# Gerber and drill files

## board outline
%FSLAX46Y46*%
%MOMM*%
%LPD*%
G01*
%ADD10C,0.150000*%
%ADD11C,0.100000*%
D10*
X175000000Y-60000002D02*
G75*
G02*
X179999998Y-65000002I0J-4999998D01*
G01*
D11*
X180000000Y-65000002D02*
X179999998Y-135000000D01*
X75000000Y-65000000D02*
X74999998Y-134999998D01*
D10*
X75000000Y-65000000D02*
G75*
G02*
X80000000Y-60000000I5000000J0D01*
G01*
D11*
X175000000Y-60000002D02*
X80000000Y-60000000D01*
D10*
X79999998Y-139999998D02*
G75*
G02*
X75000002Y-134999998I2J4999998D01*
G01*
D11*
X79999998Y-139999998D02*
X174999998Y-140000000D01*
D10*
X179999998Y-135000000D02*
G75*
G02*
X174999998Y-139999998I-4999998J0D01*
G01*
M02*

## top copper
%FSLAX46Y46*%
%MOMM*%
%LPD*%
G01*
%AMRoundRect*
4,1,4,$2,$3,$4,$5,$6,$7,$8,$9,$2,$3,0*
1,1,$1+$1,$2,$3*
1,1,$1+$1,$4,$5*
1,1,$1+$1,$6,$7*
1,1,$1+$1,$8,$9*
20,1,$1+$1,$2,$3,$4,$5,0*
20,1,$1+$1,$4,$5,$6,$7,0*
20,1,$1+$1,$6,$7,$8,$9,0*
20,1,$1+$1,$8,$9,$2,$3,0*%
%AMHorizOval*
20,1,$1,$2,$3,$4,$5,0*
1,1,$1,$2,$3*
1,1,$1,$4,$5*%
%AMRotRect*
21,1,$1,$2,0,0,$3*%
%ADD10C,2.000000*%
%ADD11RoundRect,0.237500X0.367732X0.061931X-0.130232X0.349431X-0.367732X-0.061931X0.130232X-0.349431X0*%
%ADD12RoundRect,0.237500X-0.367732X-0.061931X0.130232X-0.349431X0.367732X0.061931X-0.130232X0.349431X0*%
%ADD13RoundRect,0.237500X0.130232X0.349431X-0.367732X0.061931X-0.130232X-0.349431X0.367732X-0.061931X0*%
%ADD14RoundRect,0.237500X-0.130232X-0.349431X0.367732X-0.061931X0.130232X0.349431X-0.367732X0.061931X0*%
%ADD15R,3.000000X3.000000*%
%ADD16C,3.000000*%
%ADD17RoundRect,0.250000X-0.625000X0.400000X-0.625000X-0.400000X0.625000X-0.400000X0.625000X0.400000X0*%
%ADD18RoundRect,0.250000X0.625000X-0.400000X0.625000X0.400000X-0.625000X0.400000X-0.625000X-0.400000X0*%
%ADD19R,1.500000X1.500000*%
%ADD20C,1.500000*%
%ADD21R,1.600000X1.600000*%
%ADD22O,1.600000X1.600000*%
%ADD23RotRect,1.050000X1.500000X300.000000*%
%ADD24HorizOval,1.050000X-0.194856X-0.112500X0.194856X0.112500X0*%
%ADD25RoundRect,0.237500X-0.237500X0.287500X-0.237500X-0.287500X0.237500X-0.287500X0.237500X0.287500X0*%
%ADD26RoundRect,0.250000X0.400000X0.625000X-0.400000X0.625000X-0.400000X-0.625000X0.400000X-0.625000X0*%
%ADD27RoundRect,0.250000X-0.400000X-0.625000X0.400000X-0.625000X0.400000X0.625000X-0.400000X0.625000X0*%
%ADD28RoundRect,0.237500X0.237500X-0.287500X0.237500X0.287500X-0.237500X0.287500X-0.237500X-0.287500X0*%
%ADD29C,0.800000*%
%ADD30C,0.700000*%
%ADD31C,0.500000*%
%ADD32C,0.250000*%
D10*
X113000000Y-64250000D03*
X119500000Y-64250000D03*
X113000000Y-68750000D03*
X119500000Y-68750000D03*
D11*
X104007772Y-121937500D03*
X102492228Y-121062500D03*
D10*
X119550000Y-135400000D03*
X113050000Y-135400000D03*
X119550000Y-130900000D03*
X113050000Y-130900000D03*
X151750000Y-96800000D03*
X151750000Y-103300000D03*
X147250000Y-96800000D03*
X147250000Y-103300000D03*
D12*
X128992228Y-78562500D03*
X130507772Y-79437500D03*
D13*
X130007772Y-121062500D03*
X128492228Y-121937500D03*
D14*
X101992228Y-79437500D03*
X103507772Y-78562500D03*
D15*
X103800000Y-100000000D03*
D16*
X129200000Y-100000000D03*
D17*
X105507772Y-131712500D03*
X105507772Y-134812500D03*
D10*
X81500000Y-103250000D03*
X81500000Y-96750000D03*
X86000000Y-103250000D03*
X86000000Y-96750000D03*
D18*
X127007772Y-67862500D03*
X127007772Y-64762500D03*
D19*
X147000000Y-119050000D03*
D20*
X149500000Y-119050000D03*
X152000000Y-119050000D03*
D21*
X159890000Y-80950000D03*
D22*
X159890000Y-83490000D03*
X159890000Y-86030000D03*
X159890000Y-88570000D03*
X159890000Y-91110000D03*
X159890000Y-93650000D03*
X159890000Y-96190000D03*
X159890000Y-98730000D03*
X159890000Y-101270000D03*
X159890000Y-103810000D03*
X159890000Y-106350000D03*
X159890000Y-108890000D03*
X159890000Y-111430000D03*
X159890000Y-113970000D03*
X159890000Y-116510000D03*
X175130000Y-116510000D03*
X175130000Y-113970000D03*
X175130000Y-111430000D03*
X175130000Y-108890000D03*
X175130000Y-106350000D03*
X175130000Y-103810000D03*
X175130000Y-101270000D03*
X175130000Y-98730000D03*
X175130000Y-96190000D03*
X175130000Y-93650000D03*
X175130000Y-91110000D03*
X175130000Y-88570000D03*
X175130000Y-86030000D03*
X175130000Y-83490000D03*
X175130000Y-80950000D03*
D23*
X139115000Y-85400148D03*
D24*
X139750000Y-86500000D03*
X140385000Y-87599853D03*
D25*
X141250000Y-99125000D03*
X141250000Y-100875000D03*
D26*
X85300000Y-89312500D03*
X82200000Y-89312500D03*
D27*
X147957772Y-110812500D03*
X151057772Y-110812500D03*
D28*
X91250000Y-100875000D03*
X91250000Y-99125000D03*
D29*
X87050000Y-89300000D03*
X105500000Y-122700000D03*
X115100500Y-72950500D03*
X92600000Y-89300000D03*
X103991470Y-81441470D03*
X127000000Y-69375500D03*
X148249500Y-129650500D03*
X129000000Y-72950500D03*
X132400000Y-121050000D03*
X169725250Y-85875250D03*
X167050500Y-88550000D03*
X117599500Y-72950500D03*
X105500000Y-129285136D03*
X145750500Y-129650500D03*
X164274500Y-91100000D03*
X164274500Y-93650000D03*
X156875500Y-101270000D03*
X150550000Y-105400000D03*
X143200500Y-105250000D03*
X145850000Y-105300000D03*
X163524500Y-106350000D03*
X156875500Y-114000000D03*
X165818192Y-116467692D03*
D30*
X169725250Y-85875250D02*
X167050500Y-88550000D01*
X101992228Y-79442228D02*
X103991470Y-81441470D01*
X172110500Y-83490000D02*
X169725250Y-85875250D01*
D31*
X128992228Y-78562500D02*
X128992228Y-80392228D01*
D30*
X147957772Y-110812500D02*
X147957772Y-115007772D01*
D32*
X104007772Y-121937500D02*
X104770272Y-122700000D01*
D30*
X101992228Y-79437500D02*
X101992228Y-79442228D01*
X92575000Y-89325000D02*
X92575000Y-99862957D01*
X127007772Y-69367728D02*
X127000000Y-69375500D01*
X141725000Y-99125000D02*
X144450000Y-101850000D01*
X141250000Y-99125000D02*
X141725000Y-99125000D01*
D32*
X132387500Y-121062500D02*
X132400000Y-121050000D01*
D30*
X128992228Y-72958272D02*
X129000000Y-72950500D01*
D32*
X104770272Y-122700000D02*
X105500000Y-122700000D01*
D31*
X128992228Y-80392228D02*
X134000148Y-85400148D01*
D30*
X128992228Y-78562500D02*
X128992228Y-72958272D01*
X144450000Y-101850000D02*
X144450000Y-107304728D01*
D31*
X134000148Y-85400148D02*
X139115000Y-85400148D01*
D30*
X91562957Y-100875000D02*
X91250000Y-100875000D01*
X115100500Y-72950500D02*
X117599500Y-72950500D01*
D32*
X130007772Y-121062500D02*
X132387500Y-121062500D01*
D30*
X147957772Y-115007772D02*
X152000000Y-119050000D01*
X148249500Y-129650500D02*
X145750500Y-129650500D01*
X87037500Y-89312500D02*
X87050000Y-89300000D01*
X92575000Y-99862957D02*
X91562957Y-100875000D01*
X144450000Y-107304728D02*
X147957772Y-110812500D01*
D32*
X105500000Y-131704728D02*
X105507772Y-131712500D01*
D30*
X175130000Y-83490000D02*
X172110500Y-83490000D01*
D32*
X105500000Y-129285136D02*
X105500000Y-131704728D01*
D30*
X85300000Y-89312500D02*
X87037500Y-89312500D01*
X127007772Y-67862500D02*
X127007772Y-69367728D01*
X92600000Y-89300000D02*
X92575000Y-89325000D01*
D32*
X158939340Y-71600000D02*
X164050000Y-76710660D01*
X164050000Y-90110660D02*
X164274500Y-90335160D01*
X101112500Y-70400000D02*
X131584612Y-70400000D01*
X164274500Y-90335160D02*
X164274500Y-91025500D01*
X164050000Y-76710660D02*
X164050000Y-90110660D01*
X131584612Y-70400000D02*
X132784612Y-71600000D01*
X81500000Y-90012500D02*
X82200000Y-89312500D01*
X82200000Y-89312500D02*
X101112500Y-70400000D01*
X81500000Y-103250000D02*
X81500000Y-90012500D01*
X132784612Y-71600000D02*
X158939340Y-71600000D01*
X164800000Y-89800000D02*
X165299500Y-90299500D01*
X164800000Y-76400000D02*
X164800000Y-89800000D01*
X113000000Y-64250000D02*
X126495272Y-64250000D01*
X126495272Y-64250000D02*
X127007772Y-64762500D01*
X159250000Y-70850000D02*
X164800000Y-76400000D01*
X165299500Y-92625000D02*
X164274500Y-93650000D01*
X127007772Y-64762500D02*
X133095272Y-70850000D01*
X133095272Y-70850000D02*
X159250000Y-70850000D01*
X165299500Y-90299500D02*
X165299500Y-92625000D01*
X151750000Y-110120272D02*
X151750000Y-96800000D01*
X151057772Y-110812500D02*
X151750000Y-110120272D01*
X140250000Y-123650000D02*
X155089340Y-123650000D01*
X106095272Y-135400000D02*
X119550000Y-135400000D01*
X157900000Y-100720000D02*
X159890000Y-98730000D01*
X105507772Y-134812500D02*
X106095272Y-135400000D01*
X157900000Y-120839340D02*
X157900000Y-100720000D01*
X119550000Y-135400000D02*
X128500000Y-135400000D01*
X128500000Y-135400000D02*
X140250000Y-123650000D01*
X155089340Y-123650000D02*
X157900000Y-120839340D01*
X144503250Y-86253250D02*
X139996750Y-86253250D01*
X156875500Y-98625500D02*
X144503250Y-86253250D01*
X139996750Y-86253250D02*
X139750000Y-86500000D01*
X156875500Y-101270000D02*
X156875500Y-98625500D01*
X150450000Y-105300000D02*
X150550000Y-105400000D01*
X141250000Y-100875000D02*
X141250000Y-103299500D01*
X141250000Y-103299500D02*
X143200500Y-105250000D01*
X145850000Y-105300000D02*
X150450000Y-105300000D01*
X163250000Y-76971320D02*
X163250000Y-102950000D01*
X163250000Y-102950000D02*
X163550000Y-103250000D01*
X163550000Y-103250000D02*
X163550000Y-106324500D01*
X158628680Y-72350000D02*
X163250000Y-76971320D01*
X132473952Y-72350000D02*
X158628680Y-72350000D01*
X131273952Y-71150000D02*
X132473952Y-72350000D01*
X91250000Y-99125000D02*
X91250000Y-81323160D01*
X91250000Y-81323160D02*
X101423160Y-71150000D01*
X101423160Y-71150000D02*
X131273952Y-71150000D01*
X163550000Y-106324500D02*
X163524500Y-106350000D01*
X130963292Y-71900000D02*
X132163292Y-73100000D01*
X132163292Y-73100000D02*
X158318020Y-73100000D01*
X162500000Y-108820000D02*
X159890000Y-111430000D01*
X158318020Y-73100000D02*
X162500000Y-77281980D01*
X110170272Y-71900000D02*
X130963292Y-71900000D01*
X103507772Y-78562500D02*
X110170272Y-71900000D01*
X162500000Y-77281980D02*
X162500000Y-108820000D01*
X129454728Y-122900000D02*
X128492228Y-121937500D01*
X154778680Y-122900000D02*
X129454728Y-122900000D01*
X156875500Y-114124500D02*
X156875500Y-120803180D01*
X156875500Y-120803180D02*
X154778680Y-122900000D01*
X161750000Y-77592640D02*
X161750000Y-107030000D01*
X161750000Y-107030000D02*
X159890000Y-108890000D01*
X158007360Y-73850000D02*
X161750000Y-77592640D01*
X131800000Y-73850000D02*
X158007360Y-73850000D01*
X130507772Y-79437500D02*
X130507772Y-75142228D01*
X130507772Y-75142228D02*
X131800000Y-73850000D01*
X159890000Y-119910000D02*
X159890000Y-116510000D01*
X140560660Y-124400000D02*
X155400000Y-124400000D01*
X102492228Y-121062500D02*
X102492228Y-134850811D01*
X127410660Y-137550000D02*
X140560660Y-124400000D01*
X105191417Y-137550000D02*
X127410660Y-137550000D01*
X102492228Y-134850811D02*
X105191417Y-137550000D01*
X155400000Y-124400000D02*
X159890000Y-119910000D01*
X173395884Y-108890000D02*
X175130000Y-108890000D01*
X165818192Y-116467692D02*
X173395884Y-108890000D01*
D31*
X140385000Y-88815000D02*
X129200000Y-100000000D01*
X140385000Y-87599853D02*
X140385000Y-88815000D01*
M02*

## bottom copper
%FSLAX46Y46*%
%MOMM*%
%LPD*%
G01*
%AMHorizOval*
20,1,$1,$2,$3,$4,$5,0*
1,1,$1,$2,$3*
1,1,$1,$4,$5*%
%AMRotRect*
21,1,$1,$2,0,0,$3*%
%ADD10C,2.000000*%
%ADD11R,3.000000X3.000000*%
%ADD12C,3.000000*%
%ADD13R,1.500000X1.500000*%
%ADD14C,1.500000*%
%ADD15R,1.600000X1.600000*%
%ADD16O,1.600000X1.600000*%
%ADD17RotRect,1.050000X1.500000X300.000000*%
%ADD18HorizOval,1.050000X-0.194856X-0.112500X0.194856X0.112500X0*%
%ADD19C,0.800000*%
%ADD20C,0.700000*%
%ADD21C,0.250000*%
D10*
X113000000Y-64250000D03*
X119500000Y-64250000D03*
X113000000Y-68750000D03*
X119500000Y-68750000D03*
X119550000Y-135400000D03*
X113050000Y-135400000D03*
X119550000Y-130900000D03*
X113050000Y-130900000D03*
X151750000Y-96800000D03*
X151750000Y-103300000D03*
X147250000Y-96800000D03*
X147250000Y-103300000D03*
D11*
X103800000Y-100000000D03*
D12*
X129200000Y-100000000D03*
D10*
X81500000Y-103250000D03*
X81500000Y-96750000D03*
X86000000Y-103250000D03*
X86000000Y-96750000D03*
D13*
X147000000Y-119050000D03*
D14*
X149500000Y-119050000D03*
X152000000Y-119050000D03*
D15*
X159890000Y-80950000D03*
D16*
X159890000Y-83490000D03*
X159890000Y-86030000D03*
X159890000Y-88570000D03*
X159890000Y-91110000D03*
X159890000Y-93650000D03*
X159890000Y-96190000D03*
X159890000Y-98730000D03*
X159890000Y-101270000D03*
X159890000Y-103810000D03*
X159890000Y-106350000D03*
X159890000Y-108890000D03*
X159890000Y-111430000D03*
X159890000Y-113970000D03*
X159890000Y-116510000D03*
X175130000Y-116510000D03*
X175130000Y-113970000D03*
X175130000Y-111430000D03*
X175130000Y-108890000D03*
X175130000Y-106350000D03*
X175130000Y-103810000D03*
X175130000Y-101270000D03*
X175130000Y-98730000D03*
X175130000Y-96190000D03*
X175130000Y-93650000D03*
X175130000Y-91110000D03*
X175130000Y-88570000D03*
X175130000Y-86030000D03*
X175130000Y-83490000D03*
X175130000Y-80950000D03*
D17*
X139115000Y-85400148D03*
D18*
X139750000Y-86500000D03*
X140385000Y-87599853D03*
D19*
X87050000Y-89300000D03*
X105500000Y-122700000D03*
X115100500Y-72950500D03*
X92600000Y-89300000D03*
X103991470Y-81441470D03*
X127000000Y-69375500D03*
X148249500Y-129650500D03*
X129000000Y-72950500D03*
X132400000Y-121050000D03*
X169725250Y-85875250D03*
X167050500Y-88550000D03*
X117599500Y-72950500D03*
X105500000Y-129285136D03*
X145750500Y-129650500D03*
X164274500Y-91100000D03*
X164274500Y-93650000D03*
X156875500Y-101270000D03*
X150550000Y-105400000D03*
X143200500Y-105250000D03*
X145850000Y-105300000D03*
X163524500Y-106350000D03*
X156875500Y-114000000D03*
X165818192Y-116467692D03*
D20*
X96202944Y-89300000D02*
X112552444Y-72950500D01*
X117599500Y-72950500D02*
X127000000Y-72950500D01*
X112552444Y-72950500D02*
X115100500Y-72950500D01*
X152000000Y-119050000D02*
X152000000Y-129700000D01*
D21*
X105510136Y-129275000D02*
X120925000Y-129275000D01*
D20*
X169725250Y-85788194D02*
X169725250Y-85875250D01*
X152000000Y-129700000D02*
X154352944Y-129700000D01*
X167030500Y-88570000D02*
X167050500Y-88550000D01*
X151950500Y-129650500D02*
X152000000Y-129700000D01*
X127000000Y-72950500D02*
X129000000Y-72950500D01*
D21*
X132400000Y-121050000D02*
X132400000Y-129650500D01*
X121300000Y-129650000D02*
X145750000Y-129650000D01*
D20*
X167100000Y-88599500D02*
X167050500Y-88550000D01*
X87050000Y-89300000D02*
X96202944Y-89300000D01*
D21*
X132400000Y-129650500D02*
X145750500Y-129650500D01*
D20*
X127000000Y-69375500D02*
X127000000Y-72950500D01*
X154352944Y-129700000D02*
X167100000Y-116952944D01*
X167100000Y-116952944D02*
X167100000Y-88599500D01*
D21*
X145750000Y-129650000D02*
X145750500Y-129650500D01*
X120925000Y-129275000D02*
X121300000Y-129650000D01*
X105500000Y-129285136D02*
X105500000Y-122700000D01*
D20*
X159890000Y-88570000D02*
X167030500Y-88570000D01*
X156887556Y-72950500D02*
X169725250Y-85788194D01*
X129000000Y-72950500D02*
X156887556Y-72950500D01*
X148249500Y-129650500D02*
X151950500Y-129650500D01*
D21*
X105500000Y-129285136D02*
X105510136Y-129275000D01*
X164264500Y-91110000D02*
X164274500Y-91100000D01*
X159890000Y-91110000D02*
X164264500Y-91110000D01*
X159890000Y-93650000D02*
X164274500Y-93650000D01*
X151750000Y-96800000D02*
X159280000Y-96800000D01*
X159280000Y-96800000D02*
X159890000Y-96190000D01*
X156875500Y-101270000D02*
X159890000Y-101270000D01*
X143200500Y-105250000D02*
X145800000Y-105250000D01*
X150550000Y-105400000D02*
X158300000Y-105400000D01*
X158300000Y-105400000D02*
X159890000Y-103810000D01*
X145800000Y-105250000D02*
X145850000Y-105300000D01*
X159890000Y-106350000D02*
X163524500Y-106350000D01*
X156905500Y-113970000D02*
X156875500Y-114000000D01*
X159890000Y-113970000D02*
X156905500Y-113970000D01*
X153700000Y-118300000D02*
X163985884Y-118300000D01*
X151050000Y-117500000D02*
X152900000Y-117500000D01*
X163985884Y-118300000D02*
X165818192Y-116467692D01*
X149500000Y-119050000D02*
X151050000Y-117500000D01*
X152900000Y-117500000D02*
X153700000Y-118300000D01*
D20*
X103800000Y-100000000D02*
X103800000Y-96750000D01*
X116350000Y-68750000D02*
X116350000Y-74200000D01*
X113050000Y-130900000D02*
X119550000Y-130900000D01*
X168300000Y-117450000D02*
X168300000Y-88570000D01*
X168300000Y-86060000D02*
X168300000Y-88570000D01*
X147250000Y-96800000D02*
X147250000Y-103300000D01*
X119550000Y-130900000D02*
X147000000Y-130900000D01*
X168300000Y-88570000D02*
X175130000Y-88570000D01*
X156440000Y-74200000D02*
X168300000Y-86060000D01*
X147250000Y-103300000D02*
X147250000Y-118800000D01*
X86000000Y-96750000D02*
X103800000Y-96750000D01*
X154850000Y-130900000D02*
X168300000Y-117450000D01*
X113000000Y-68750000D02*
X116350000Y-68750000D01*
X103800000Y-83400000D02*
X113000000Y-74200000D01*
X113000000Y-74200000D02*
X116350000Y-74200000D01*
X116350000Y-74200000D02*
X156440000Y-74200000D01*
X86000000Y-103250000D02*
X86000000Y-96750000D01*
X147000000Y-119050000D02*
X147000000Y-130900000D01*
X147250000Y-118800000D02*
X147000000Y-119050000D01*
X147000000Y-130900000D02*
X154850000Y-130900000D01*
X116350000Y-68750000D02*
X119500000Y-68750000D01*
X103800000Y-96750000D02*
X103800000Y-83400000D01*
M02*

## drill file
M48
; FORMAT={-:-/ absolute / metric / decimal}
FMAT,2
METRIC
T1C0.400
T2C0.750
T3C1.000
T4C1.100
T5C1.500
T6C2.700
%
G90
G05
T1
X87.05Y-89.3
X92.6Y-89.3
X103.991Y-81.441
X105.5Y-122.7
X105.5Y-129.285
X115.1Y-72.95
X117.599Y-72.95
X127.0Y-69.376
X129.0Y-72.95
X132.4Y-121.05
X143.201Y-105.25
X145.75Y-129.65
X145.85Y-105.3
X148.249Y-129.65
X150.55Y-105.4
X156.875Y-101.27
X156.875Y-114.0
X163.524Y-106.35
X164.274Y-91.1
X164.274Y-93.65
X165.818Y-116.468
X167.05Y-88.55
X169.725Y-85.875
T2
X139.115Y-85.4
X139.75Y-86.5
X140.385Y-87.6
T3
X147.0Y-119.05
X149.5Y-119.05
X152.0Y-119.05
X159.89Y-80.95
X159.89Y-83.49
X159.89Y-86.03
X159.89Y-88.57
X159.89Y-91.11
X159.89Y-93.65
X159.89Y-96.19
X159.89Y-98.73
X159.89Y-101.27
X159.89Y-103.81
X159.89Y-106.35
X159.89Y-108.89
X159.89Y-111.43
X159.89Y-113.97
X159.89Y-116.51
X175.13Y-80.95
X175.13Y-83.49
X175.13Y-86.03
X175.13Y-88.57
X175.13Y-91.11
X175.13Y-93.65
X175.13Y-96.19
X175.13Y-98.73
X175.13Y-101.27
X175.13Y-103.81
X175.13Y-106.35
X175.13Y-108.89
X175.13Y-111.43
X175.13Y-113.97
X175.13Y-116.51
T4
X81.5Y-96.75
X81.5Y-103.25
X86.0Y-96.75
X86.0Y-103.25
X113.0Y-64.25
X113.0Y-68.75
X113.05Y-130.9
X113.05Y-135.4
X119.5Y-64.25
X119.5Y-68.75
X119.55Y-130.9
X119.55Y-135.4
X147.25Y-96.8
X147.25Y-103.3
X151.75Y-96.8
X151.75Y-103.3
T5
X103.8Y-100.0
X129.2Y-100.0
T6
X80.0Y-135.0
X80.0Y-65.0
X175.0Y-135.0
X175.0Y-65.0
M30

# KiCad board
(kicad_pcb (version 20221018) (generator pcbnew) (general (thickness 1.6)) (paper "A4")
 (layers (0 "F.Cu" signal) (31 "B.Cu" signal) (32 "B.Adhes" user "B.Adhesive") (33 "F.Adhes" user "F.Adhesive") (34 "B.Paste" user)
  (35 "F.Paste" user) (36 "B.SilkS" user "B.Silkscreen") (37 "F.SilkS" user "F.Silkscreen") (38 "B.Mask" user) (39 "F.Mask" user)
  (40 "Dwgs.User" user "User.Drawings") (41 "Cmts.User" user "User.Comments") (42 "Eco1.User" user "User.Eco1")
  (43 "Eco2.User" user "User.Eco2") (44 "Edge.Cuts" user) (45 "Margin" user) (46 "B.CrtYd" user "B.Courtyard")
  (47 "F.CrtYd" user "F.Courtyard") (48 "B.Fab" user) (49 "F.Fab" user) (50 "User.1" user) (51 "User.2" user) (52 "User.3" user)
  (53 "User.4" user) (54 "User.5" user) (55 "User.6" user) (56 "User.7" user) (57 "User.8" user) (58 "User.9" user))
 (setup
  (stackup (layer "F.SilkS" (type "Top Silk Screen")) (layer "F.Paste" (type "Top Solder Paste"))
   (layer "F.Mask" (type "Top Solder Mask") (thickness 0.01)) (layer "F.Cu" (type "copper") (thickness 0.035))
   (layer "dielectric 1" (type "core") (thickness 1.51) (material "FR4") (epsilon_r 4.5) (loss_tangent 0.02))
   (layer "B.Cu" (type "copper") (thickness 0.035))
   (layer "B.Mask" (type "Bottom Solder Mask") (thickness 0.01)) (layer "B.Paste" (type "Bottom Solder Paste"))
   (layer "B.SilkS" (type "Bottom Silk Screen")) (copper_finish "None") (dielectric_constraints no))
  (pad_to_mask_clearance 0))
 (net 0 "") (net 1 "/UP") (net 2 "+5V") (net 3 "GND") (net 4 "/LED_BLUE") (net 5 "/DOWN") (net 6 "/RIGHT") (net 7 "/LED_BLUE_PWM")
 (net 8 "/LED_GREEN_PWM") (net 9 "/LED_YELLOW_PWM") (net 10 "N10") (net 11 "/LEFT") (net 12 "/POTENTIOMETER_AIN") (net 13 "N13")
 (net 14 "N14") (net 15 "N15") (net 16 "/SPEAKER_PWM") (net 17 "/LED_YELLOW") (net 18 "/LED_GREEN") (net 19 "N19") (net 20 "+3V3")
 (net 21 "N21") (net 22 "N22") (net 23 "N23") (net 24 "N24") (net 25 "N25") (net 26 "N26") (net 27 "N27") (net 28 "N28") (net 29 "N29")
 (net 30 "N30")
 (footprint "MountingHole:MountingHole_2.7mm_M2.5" (layer "F.Cu") (at 80 65)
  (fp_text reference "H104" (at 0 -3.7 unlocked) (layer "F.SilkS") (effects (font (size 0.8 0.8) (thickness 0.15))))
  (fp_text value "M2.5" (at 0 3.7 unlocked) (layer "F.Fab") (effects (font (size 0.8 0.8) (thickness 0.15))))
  (pad "" np_thru_hole circle (at 0 0) (size 2.7 2.7) (drill 2.7) (layers "*.Cu" "*.Mask")))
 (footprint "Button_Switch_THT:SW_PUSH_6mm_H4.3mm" (layer "F.Cu") (at 113 64.25)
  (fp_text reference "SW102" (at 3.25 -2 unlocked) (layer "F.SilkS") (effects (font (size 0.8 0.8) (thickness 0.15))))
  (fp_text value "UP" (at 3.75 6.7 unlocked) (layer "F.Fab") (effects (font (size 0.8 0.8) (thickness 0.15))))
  (pad "1" thru_hole circle (at 0 0 90) (size 2 2) (drill 1.1) (layers "*.Cu" "*.Mask") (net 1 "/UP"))
  (pad "1" thru_hole circle (at 6.5 0 90) (size 2 2) (drill 1.1) (layers "*.Cu" "*.Mask") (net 1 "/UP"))
  (pad "2" thru_hole circle (at 0 4.5 90) (size 2 2) (drill 1.1) (layers "*.Cu" "*.Mask") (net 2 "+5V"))
  (pad "2" thru_hole circle (at 6.5 4.5 90) (size 2 2) (drill 1.1) (layers "*.Cu" "*.Mask") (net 2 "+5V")))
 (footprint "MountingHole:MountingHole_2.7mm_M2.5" (layer "F.Cu") (at 175 65.000002)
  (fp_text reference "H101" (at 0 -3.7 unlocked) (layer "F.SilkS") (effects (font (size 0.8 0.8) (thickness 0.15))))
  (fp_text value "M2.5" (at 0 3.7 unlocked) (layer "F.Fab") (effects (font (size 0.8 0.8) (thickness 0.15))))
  (pad "" np_thru_hole circle (at 0 0) (size 2.7 2.7) (drill 2.7) (layers "*.Cu" "*.Mask")))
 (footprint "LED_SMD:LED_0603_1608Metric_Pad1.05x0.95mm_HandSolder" (layer "F.Cu") (at 103.25 121.5 150)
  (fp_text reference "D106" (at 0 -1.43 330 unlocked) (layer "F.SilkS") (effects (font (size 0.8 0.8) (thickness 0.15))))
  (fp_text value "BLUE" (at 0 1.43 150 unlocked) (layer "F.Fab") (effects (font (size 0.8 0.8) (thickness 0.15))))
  (pad "1" smd roundrect (at -0.875 0 150) (size 1.05 0.95) (layers "F.Cu" "F.Paste" "F.Mask") (roundrect_rratio 0.25) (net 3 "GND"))
  (pad "2" smd roundrect (at 0.875 0 150) (size 1.05 0.95) (layers "F.Cu" "F.Paste" "F.Mask") (roundrect_rratio 0.25) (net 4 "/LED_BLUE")))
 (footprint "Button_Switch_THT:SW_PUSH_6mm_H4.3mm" (layer "F.Cu") (at 119.55 135.4 180)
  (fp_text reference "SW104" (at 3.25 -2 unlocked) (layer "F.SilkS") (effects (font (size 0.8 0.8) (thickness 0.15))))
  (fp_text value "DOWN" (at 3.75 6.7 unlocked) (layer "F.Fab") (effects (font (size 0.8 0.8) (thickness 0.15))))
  (pad "1" thru_hole circle (at 0 0 270) (size 2 2) (drill 1.1) (layers "*.Cu" "*.Mask") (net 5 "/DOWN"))
  (pad "1" thru_hole circle (at 6.5 0 270) (size 2 2) (drill 1.1) (layers "*.Cu" "*.Mask") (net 5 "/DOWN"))
  (pad "2" thru_hole circle (at 0 4.5 270) (size 2 2) (drill 1.1) (layers "*.Cu" "*.Mask") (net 2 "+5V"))
  (pad "2" thru_hole circle (at 6.5 4.5 270) (size 2 2) (drill 1.1) (layers "*.Cu" "*.Mask") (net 2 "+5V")))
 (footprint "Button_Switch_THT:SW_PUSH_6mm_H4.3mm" (layer "F.Cu") (at 151.75 96.8 -90)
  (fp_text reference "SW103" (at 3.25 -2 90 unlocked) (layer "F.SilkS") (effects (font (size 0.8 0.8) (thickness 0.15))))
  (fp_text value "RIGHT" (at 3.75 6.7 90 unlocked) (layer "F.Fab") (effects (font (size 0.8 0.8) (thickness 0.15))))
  (pad "1" thru_hole circle (at 0 0) (size 2 2) (drill 1.1) (layers "*.Cu" "*.Mask") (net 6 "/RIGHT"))
  (pad "1" thru_hole circle (at 6.5 0) (size 2 2) (drill 1.1) (layers "*.Cu" "*.Mask") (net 6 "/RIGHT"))
  (pad "2" thru_hole circle (at 0 4.5) (size 2 2) (drill 1.1) (layers "*.Cu" "*.Mask") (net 2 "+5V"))
  (pad "2" thru_hole circle (at 6.5 4.5) (size 2 2) (drill 1.1) (layers "*.Cu" "*.Mask") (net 2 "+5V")))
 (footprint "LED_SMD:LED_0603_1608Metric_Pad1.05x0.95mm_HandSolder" (layer "F.Cu") (at 129.75 79 -30)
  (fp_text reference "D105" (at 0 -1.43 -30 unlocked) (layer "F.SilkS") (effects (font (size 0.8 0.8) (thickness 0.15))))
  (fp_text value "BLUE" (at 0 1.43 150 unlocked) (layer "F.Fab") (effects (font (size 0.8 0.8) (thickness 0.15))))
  (pad "1" smd roundrect (at -0.875 0 330) (size 1.05 0.95) (layers "F.Cu" "F.Paste" "F.Mask") (roundrect_rratio 0.25) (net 3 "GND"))
  (pad "2" smd roundrect (at 0.875 0 330) (size 1.05 0.95) (layers "F.Cu" "F.Paste" "F.Mask") (roundrect_rratio 0.25)
   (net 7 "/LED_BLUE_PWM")))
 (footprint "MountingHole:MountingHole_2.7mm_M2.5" (layer "F.Cu") (at 174.999998 135)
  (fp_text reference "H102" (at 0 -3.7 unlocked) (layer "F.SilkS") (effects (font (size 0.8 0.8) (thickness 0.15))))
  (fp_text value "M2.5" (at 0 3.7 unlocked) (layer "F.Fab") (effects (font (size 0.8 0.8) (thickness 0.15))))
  (pad "" np_thru_hole circle (at 0 0) (size 2.7 2.7) (drill 2.7) (layers "*.Cu" "*.Mask")))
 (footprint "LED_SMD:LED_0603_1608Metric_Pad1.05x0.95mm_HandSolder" (layer "F.Cu") (at 129.25 121.5 -150)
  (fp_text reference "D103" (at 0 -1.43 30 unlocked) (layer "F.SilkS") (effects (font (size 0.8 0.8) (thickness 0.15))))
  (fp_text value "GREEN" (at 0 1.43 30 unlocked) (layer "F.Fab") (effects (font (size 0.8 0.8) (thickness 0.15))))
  (pad "1" smd roundrect (at -0.875 0 210) (size 1.05 0.95) (layers "F.Cu" "F.Paste" "F.Mask") (roundrect_rratio 0.25) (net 3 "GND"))
  (pad "2" smd roundrect (at 0.875 0 210) (size 1.05 0.95) (layers "F.Cu" "F.Paste" "F.Mask") (roundrect_rratio 0.25)
   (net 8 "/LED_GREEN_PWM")))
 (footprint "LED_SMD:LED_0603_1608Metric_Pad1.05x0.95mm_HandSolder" (layer "F.Cu") (at 102.75 79 30)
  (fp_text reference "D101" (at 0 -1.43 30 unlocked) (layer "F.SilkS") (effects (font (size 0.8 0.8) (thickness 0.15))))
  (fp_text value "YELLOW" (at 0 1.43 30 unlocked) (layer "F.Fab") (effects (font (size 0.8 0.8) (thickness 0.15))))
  (pad "1" smd roundrect (at -0.875 0 30) (size 1.05 0.95) (layers "F.Cu" "F.Paste" "F.Mask") (roundrect_rratio 0.25) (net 3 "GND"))
  (pad "2" smd roundrect (at 0.875 0 30) (size 1.05 0.95) (layers "F.Cu" "F.Paste" "F.Mask") (roundrect_rratio 0.25)
   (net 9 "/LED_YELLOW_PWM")))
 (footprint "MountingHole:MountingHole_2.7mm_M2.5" (layer "F.Cu") (at 79.999998 134.999998)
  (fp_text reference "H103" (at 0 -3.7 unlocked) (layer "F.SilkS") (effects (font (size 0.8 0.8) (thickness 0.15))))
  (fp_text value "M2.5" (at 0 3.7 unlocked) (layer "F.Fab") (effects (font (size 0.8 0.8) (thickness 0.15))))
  (pad "" np_thru_hole circle (at 0 0) (size 2.7 2.7) (drill 2.7) (layers "*.Cu" "*.Mask")))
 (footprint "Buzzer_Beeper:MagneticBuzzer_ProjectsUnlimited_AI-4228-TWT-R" (layer "F.Cu") (at 103.8 100)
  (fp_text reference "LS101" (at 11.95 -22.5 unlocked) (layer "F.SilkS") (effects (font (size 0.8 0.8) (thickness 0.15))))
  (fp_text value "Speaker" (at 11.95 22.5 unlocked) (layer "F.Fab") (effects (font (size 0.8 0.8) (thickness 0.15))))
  (pad "1" thru_hole rect (at 0 0) (size 3 3) (drill 1.5) (layers "*.Cu" "*.Mask") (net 2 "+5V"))
  (pad "2" thru_hole circle (at 25.4 0) (size 3 3) (drill 1.5) (layers "*.Cu" "*.Mask") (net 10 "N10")))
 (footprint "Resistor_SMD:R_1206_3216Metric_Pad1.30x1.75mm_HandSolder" (layer "F.Cu") (at 105.507772 133.2625 -90)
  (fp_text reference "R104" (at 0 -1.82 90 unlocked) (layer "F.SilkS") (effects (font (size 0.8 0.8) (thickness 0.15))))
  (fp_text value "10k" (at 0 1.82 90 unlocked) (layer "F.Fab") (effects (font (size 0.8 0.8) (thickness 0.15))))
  (pad "1" smd roundrect (at -1.55 0 270) (size 1.3 1.75) (layers "F.Cu" "F.Paste" "F.Mask") (roundrect_rratio 0.1923076923) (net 3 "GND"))
  (pad "2" smd roundrect (at 1.55 0 270) (size 1.3 1.75) (layers "F.Cu" "F.Paste" "F.Mask") (roundrect_rratio 0.1923076923) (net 5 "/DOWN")))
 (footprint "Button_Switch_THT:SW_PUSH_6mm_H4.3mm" (layer "F.Cu") (at 81.5 103.25 90)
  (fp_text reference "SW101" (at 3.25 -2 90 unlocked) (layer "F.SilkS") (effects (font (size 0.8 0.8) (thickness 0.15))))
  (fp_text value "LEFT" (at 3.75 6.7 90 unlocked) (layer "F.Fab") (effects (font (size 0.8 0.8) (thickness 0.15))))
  (pad "1" thru_hole circle (at 0 0 180) (size 2 2) (drill 1.1) (layers "*.Cu" "*.Mask") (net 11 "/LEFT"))
  (pad "1" thru_hole circle (at 6.5 0 180) (size 2 2) (drill 1.1) (layers "*.Cu" "*.Mask") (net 11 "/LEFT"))
  (pad "2" thru_hole circle (at 0 4.5 180) (size 2 2) (drill 1.1) (layers "*.Cu" "*.Mask") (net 2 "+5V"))
  (pad "2" thru_hole circle (at 6.5 4.5 180) (size 2 2) (drill 1.1) (layers "*.Cu" "*.Mask") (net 2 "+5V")))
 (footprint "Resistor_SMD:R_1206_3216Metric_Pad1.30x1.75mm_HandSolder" (layer "F.Cu") (at 127.007772 66.3125 90)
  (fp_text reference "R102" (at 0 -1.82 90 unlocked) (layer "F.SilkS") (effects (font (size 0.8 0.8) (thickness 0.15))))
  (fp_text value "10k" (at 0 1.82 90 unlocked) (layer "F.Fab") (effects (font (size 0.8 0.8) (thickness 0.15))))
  (pad "1" smd roundrect (at -1.55 0 90) (size 1.3 1.75) (layers "F.Cu" "F.Paste" "F.Mask") (roundrect_rratio 0.1923076923) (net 3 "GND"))
  (pad "2" smd roundrect (at 1.55 0 90) (size 1.3 1.75) (layers "F.Cu" "F.Paste" "F.Mask") (roundrect_rratio 0.1923076923) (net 1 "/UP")))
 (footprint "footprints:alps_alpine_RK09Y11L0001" (layer "F.Cu") (at 147 119.05 90)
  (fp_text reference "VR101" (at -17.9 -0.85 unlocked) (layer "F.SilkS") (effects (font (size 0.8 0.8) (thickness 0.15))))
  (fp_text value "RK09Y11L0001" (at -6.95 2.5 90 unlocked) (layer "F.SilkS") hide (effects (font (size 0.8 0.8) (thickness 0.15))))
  (pad "1" thru_hole rect (at 0 0 90) (size 1.5 1.5) (drill 1) (layers "*.Cu" "*.Mask") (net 2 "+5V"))
  (pad "2" thru_hole circle (at 0 2.5 90) (size 1.5 1.5) (drill 1) (layers "*.Cu" "*.Mask") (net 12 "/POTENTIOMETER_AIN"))
  (pad "3" thru_hole circle (at 0 5 90) (size 1.5 1.5) (drill 1) (layers "*.Cu" "*.Mask") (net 3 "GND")))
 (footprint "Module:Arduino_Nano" (layer "F.Cu") (at 159.89 80.95)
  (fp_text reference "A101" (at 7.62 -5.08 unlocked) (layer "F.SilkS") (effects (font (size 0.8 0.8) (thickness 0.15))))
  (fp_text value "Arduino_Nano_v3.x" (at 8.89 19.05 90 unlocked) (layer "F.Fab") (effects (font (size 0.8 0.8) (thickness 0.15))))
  (pad "1" thru_hole rect (at 0 0) (size 1.6 1.6) (drill 1) (layers "*.Cu" "*.Mask") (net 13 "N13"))
  (pad "2" thru_hole oval (at 0 2.54) (size 1.6 1.6) (drill 1) (layers "*.Cu" "*.Mask") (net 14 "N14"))
  (pad "3" thru_hole oval (at 0 5.08) (size 1.6 1.6) (drill 1) (layers "*.Cu" "*.Mask") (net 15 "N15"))
  (pad "4" thru_hole oval (at 0 7.62) (size 1.6 1.6) (drill 1) (layers "*.Cu" "*.Mask") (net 3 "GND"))
  (pad "5" thru_hole oval (at 0 10.16) (size 1.6 1.6) (drill 1) (layers "*.Cu" "*.Mask") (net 11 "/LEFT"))
  (pad "6" thru_hole oval (at 0 12.7) (size 1.6 1.6) (drill 1) (layers "*.Cu" "*.Mask") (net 1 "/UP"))
  (pad "7" thru_hole oval (at 0 15.24) (size 1.6 1.6) (drill 1) (layers "*.Cu" "*.Mask") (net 6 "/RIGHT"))
  (pad "8" thru_hole oval (at 0 17.78) (size 1.6 1.6) (drill 1) (layers "*.Cu" "*.Mask") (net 5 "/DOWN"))
  (pad "9" thru_hole oval (at 0 20.32) (size 1.6 1.6) (drill 1) (layers "*.Cu" "*.Mask") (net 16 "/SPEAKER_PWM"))
  (pad "10" thru_hole oval (at 0 22.86) (size 1.6 1.6) (drill 1) (layers "*.Cu" "*.Mask") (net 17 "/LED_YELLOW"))
  (pad "11" thru_hole oval (at 0 25.4) (size 1.6 1.6) (drill 1) (layers "*.Cu" "*.Mask") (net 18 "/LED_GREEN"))
  (pad "12" thru_hole oval (at 0 27.94) (size 1.6 1.6) (drill 1) (layers "*.Cu" "*.Mask") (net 7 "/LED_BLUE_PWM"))
  (pad "13" thru_hole oval (at 0 30.48) (size 1.6 1.6) (drill 1) (layers "*.Cu" "*.Mask") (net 9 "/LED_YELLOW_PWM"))
  (pad "14" thru_hole oval (at 0 33.02) (size 1.6 1.6) (drill 1) (layers "*.Cu" "*.Mask") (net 8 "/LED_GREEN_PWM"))
  (pad "15" thru_hole oval (at 0 35.56) (size 1.6 1.6) (drill 1) (layers "*.Cu" "*.Mask") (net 4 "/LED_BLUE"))
  (pad "16" thru_hole oval (at 15.24 35.56) (size 1.6 1.6) (drill 1) (layers "*.Cu" "*.Mask") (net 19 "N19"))
  (pad "17" thru_hole oval (at 15.24 33.02) (size 1.6 1.6) (drill 1) (layers "*.Cu" "*.Mask") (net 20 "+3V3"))
  (pad "18" thru_hole oval (at 15.24 30.48) (size 1.6 1.6) (drill 1) (layers "*.Cu" "*.Mask") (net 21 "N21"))
  (pad "19" thru_hole oval (at 15.24 27.94) (size 1.6 1.6) (drill 1) (layers "*.Cu" "*.Mask") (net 12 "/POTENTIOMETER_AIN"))
  (pad "20" thru_hole oval (at 15.24 25.4) (size 1.6 1.6) (drill 1) (layers "*.Cu" "*.Mask") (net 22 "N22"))
  (pad "21" thru_hole oval (at 15.24 22.86) (size 1.6 1.6) (drill 1) (layers "*.Cu" "*.Mask") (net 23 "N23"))
  (pad "22" thru_hole oval (at 15.24 20.32) (size 1.6 1.6) (drill 1) (layers "*.Cu" "*.Mask") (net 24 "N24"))
  (pad "23" thru_hole oval (at 15.24 17.78) (size 1.6 1.6) (drill 1) (layers "*.Cu" "*.Mask") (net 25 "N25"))
  (pad "24" thru_hole oval (at 15.24 15.24) (size 1.6 1.6) (drill 1) (layers "*.Cu" "*.Mask") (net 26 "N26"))
  (pad "25" thru_hole oval (at 15.24 12.7) (size 1.6 1.6) (drill 1) (layers "*.Cu" "*.Mask") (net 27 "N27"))
  (pad "26" thru_hole oval (at 15.24 10.16) (size 1.6 1.6) (drill 1) (layers "*.Cu" "*.Mask") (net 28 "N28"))
  (pad "27" thru_hole oval (at 15.24 7.62) (size 1.6 1.6) (drill 1) (layers "*.Cu" "*.Mask") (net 2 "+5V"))
  (pad "28" thru_hole oval (at 15.24 5.08) (size 1.6 1.6) (drill 1) (layers "*.Cu" "*.Mask") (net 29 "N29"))
  (pad "29" thru_hole oval (at 15.24 2.54) (size 1.6 1.6) (drill 1) (layers "*.Cu" "*.Mask") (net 3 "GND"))
  (pad "30" thru_hole oval (at 15.24 0) (size 1.6 1.6) (drill 1) (layers "*.Cu" "*.Mask") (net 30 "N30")))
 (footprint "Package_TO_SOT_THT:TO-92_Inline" (layer "F.Cu") (at 139.115 85.400148 -60)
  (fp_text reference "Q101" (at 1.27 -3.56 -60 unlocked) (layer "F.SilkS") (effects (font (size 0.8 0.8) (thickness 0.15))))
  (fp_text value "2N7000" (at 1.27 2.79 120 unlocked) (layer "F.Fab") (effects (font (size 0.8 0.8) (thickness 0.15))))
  (pad "1" thru_hole rect (at 0 0 300) (size 1.05 1.5) (drill 0.75) (layers "*.Cu" "*.Mask") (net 3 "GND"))
  (pad "2" thru_hole oval (at 1.27 0 300) (size 1.05 1.5) (drill 0.75) (layers "*.Cu" "*.Mask") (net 16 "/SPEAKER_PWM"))
  (pad "3" thru_hole oval (at 2.54 0 300) (size 1.05 1.5) (drill 0.75) (layers "*.Cu" "*.Mask") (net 10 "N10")))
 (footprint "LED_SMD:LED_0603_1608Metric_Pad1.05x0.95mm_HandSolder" (layer "F.Cu") (at 141.25 100 -90)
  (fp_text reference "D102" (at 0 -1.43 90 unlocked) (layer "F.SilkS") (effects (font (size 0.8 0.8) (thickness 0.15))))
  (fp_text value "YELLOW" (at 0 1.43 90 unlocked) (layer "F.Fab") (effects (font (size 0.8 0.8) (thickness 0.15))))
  (pad "1" smd roundrect (at -0.875 0 270) (size 1.05 0.95) (layers "F.Cu" "F.Paste" "F.Mask") (roundrect_rratio 0.25) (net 3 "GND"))
  (pad "2" smd roundrect (at 0.875 0 270) (size 1.05 0.95) (layers "F.Cu" "F.Paste" "F.Mask") (roundrect_rratio 0.25) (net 17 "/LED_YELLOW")))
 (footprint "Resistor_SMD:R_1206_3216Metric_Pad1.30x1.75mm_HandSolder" (layer "F.Cu") (at 83.75 89.3125 180)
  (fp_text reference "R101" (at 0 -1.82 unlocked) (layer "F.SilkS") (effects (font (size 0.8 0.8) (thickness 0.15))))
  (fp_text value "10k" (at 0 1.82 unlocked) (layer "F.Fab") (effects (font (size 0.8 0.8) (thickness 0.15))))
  (pad "1" smd roundrect (at -1.55 0 180) (size 1.3 1.75) (layers "F.Cu" "F.Paste" "F.Mask") (roundrect_rratio 0.1923076923) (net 3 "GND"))
  (pad "2" smd roundrect (at 1.55 0 180) (size 1.3 1.75) (layers "F.Cu" "F.Paste" "F.Mask") (roundrect_rratio 0.1923076923) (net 11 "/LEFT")))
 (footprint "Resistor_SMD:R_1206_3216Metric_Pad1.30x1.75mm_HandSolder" (layer "F.Cu") (at 149.507772 110.8125)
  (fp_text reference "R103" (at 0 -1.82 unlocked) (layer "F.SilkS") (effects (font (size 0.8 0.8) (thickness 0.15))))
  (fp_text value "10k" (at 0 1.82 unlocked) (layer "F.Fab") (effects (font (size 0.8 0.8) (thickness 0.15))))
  (pad "1" smd roundrect (at -1.55 0) (size 1.3 1.75) (layers "F.Cu" "F.Paste" "F.Mask") (roundrect_rratio 0.1923076923) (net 3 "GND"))
  (pad "2" smd roundrect (at 1.55 0) (size 1.3 1.75) (layers "F.Cu" "F.Paste" "F.Mask") (roundrect_rratio 0.1923076923) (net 6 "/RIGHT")))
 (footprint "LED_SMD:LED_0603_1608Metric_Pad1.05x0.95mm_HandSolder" (layer "F.Cu") (at 91.25 100 90)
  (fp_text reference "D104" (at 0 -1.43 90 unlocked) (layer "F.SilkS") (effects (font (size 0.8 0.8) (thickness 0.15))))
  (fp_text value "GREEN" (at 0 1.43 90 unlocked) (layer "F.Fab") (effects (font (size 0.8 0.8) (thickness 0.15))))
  (pad "1" smd roundrect (at -0.875 0 90) (size 1.05 0.95) (layers "F.Cu" "F.Paste" "F.Mask") (roundrect_rratio 0.25) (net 3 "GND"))
  (pad "2" smd roundrect (at 0.875 0 90) (size 1.05 0.95) (layers "F.Cu" "F.Paste" "F.Mask") (roundrect_rratio 0.25) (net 18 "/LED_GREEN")))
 (gr_arc (start 175 60.000002) (mid 178.535533 61.464468) (end 180 65.000002) (stroke (width 0.15) (type default)) (layer "Edge.Cuts"))
 (gr_line (start 180 65.000002) (end 179.999998 135) (stroke (width 0.1) (type default)) (layer "Edge.Cuts"))
 (gr_line (start 75 65) (end 74.999998 134.999998) (stroke (width 0.1) (type default)) (layer "Edge.Cuts"))
 (gr_arc (start 75 65) (mid 76.464466 61.464467) (end 80 60) (stroke (width 0.15) (type default)) (layer "Edge.Cuts"))
 (gr_line (start 175 60.000002) (end 80 60) (stroke (width 0.1) (type default)) (layer "Edge.Cuts"))
 (gr_arc (start 79.999998 139.999998) (mid 76.464465 138.535532) (end 74.999998 134.999998) (stroke (width 0.15) (type default))
  (layer "Edge.Cuts"))
 (gr_line (start 79.999998 139.999998) (end 174.999998 140) (stroke (width 0.1) (type default)) (layer "Edge.Cuts"))
 (gr_arc (start 179.999998 135) (mid 178.535532 138.535533) (end 174.999998 140) (stroke (width 0.15) (type default)) (layer "Edge.Cuts"))
 (segment (start 169.72525 85.87525) (end 167.0505 88.55) (width 0.7) (layer "F.Cu") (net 3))
 (segment (start 101.992228 79.442228) (end 103.99147 81.44147) (width 0.7) (layer "F.Cu") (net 3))
 (segment (start 172.1105 83.49) (end 169.72525 85.87525) (width 0.7) (layer "F.Cu") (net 3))
 (segment (start 128.992228 78.5625) (end 128.992228 80.392228) (width 0.5) (layer "F.Cu") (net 3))
 (segment (start 147.957772 110.8125) (end 147.957772 115.007772) (width 0.7) (layer "F.Cu") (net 3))
 (segment (start 104.007772 121.9375) (end 104.770272 122.7) (width 0.25) (layer "F.Cu") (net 3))
 (segment (start 101.992228 79.4375) (end 101.992228 79.442228) (width 0.7) (layer "F.Cu") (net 3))
 (segment (start 92.575 89.325) (end 92.575 99.862957) (width 0.7) (layer "F.Cu") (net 3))
 (segment (start 127.007772 69.367728) (end 127 69.3755) (width 0.7) (layer "F.Cu") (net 3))
 (segment (start 141.725 99.125) (end 144.45 101.85) (width 0.7) (layer "F.Cu") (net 3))
 (segment (start 141.25 99.125) (end 141.725 99.125) (width 0.7) (layer "F.Cu") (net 3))
 (segment (start 132.3875 121.0625) (end 132.4 121.05) (width 0.25) (layer "F.Cu") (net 3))
 (segment (start 128.992228 72.958272) (end 129 72.9505) (width 0.7) (layer "F.Cu") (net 3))
 (segment (start 104.770272 122.7) (end 105.5 122.7) (width 0.25) (layer "F.Cu") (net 3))
 (segment (start 128.992228 80.392228) (end 134.000148 85.400148) (width 0.5) (layer "F.Cu") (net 3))
 (segment (start 128.992228 78.5625) (end 128.992228 72.958272) (width 0.7) (layer "F.Cu") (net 3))
 (segment (start 144.45 101.85) (end 144.45 107.304728) (width 0.7) (layer "F.Cu") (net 3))
 (segment (start 134.000148 85.400148) (end 139.115 85.400148) (width 0.5) (layer "F.Cu") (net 3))
 (segment (start 91.562957 100.875) (end 91.25 100.875) (width 0.7) (layer "F.Cu") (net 3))
 (segment (start 115.1005 72.9505) (end 117.5995 72.9505) (width 0.7) (layer "F.Cu") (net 3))
 (segment (start 130.007772 121.0625) (end 132.3875 121.0625) (width 0.25) (layer "F.Cu") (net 3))
 (segment (start 147.957772 115.007772) (end 152 119.05) (width 0.7) (layer "F.Cu") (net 3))
 (segment (start 148.2495 129.6505) (end 145.7505 129.6505) (width 0.7) (layer "F.Cu") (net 3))
 (segment (start 87.0375 89.3125) (end 87.05 89.3) (width 0.7) (layer "F.Cu") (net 3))
 (segment (start 92.575 99.862957) (end 91.562957 100.875) (width 0.7) (layer "F.Cu") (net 3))
 (segment (start 144.45 107.304728) (end 147.957772 110.8125) (width 0.7) (layer "F.Cu") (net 3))
 (segment (start 105.5 131.704728) (end 105.507772 131.7125) (width 0.25) (layer "F.Cu") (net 3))
 (segment (start 175.13 83.49) (end 172.1105 83.49) (width 0.7) (layer "F.Cu") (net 3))
 (segment (start 105.5 129.285136) (end 105.5 131.704728) (width 0.25) (layer "F.Cu") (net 3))
 (segment (start 85.3 89.3125) (end 87.0375 89.3125) (width 0.7) (layer "F.Cu") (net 3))
 (segment (start 127.007772 67.8625) (end 127.007772 69.367728) (width 0.7) (layer "F.Cu") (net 3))
 (segment (start 92.6 89.3) (end 92.575 89.325) (width 0.7) (layer "F.Cu") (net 3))
 (via (at 87.05 89.3) (size 0.8) (drill 0.4) (layers "F.Cu" "B.Cu") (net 3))
 (via (at 105.5 122.7) (size 0.8) (drill 0.4) (layers "F.Cu" "B.Cu") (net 3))
 (via (at 115.1005 72.9505) (size 0.8) (drill 0.4) (layers "F.Cu" "B.Cu") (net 3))
 (via (at 92.6 89.3) (size 0.8) (drill 0.4) (layers "F.Cu" "B.Cu") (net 3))
 (via (at 103.99147 81.44147) (size 0.8) (drill 0.4) (layers "F.Cu" "B.Cu") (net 3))
 (via (at 127 69.3755) (size 0.8) (drill 0.4) (layers "F.Cu" "B.Cu") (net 3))
 (via (at 148.2495 129.6505) (size 0.8) (drill 0.4) (layers "F.Cu" "B.Cu") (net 3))
 (via (at 129 72.9505) (size 0.8) (drill 0.4) (layers "F.Cu" "B.Cu") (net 3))
 (via (at 132.4 121.05) (size 0.8) (drill 0.4) (layers "F.Cu" "B.Cu") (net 3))
 (via (at 169.72525 85.87525) (size 0.8) (drill 0.4) (layers "F.Cu" "B.Cu") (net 3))
 (via (at 167.0505 88.55) (size 0.8) (drill 0.4) (layers "F.Cu" "B.Cu") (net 3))
 (via (at 117.5995 72.9505) (size 0.8) (drill 0.4) (layers "F.Cu" "B.Cu") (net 3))
 (via (at 105.5 129.285136) (size 0.8) (drill 0.4) (layers "F.Cu" "B.Cu") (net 3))
 (via (at 145.7505 129.6505) (size 0.8) (drill 0.4) (layers "F.Cu" "B.Cu") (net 3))
 (segment (start 96.202944 89.3) (end 112.552444 72.9505) (width 0.7) (layer "B.Cu") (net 3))
 (segment (start 117.5995 72.9505) (end 127 72.9505) (width 0.7) (layer "B.Cu") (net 3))
 (segment (start 112.552444 72.9505) (end 115.1005 72.9505) (width 0.7) (layer "B.Cu") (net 3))
 (segment (start 152 119.05) (end 152 129.7) (width 0.7) (layer "B.Cu") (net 3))
 (segment (start 105.510136 129.275) (end 120.925 129.275) (width 0.25) (layer "B.Cu") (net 3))
 (segment (start 169.72525 85.788194) (end 169.72525 85.87525) (width 0.7) (layer "B.Cu") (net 3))
 (segment (start 152 129.7) (end 154.352944 129.7) (width 0.7) (layer "B.Cu") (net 3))
 (segment (start 167.0305 88.57) (end 167.0505 88.55) (width 0.7) (layer "B.Cu") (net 3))
 (segment (start 151.9505 129.6505) (end 152 129.7) (width 0.7) (layer "B.Cu") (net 3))
 (segment (start 127 72.9505) (end 129 72.9505) (width 0.7) (layer "B.Cu") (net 3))
 (segment (start 132.4 121.05) (end 132.4 129.6505) (width 0.25) (layer "B.Cu") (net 3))
 (segment (start 121.3 129.65) (end 145.75 129.65) (width 0.25) (layer "B.Cu") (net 3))
 (segment (start 167.1 88.5995) (end 167.0505 88.55) (width 0.7) (layer "B.Cu") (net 3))
 (segment (start 87.05 89.3) (end 96.202944 89.3) (width 0.7) (layer "B.Cu") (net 3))
 (segment (start 132.4 129.6505) (end 145.7505 129.6505) (width 0.25) (layer "B.Cu") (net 3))
 (segment (start 127 69.3755) (end 127 72.9505) (width 0.7) (layer "B.Cu") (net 3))
 (segment (start 154.352944 129.7) (end 167.1 116.952944) (width 0.7) (layer "B.Cu") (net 3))
 (segment (start 167.1 116.952944) (end 167.1 88.5995) (width 0.7) (layer "B.Cu") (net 3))
 (segment (start 145.75 129.65) (end 145.7505 129.6505) (width 0.25) (layer "B.Cu") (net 3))
 (segment (start 120.925 129.275) (end 121.3 129.65) (width 0.25) (layer "B.Cu") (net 3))
 (segment (start 105.5 129.285136) (end 105.5 122.7) (width 0.25) (layer "B.Cu") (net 3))
 (segment (start 159.89 88.57) (end 167.0305 88.57) (width 0.7) (layer "B.Cu") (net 3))
 (segment (start 156.887556 72.9505) (end 169.72525 85.788194) (width 0.7) (layer "B.Cu") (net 3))
 (segment (start 129 72.9505) (end 156.887556 72.9505) (width 0.7) (layer "B.Cu") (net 3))
 (segment (start 148.2495 129.6505) (end 151.9505 129.6505) (width 0.7) (layer "B.Cu") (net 3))
 (segment (start 105.5 129.285136) (end 105.510136 129.275) (width 0.25) (layer "B.Cu") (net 3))
 (segment (start 158.93934 71.6) (end 164.05 76.71066) (width 0.25) (layer "F.Cu") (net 11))
 (segment (start 164.05 90.11066) (end 164.2745 90.33516) (width 0.25) (layer "F.Cu") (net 11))
 (segment (start 101.1125 70.4) (end 131.584612 70.4) (width 0.25) (layer "F.Cu") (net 11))
 (segment (start 164.2745 90.33516) (end 164.2745 91.0255) (width 0.25) (layer "F.Cu") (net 11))
 (segment (start 164.05 76.71066) (end 164.05 90.11066) (width 0.25) (layer "F.Cu") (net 11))
 (segment (start 131.584612 70.4) (end 132.784612 71.6) (width 0.25) (layer "F.Cu") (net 11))
 (segment (start 81.5 90.0125) (end 82.2 89.3125) (width 0.25) (layer "F.Cu") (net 11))
 (segment (start 82.2 89.3125) (end 101.1125 70.4) (width 0.25) (layer "F.Cu") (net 11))
 (segment (start 81.5 103.25) (end 81.5 90.0125) (width 0.25) (layer "F.Cu") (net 11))
 (segment (start 132.784612 71.6) (end 158.93934 71.6) (width 0.25) (layer "F.Cu") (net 11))
 (via (at 164.2745 91.1) (size 0.8) (drill 0.4) (layers "F.Cu" "B.Cu") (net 11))
 (segment (start 164.2645 91.11) (end 164.2745 91.1) (width 0.25) (layer "B.Cu") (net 11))
 (segment (start 159.89 91.11) (end 164.2645 91.11) (width 0.25) (layer "B.Cu") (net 11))
 (segment (start 164.8 89.8) (end 165.2995 90.2995) (width 0.25) (layer "F.Cu") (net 1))
 (segment (start 164.8 76.4) (end 164.8 89.8) (width 0.25) (layer "F.Cu") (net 1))
 (segment (start 113 64.25) (end 126.495272 64.25) (width 0.25) (layer "F.Cu") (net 1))
 (segment (start 126.495272 64.25) (end 127.007772 64.7625) (width 0.25) (layer "F.Cu") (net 1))
 (segment (start 159.25 70.85) (end 164.8 76.4) (width 0.25) (layer "F.Cu") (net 1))
 (segment (start 165.2995 92.625) (end 164.2745 93.65) (width 0.25) (layer "F.Cu") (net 1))
 (segment (start 127.007772 64.7625) (end 133.095272 70.85) (width 0.25) (layer "F.Cu") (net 1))
 (segment (start 133.095272 70.85) (end 159.25 70.85) (width 0.25) (layer "F.Cu") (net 1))
 (segment (start 165.2995 90.2995) (end 165.2995 92.625) (width 0.25) (layer "F.Cu") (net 1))
 (via (at 164.2745 93.65) (size 0.8) (drill 0.4) (layers "F.Cu" "B.Cu") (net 1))
 (segment (start 159.89 93.65) (end 164.2745 93.65) (width 0.25) (layer "B.Cu") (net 1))
 (segment (start 151.75 110.120272) (end 151.75 96.8) (width 0.25) (layer "F.Cu") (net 6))
 (segment (start 151.057772 110.8125) (end 151.75 110.120272) (width 0.25) (layer "F.Cu") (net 6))
 (segment (start 151.75 96.8) (end 159.28 96.8) (width 0.25) (layer "B.Cu") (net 6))
 (segment (start 159.28 96.8) (end 159.89 96.19) (width 0.25) (layer "B.Cu") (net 6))
 (segment (start 140.25 123.65) (end 155.08934 123.65) (width 0.25) (layer "F.Cu") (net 5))
 (segment (start 106.095272 135.4) (end 119.55 135.4) (width 0.25) (layer "F.Cu") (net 5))
 (segment (start 157.9 100.72) (end 159.89 98.73) (width 0.25) (layer "F.Cu") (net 5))
 (segment (start 105.507772 134.8125) (end 106.095272 135.4) (width 0.25) (layer "F.Cu") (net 5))
 (segment (start 157.9 120.83934) (end 157.9 100.72) (width 0.25) (layer "F.Cu") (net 5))
 (segment (start 119.55 135.4) (end 128.5 135.4) (width 0.25) (layer "F.Cu") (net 5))
 (segment (start 128.5 135.4) (end 140.25 123.65) (width 0.25) (layer "F.Cu") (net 5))
 (segment (start 155.08934 123.65) (end 157.9 120.83934) (width 0.25) (layer "F.Cu") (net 5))
 (segment (start 144.50325 86.25325) (end 139.99675 86.25325) (width 0.25) (layer "F.Cu") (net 16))
 (segment (start 156.8755 98.6255) (end 144.50325 86.25325) (width 0.25) (layer "F.Cu") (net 16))
 (segment (start 139.99675 86.25325) (end 139.75 86.5) (width 0.25) (layer "F.Cu") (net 16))
 (segment (start 156.8755 101.27) (end 156.8755 98.6255) (width 0.25) (layer "F.Cu") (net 16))
 (via (at 156.8755 101.27) (size 0.8) (drill 0.4) (layers "F.Cu" "B.Cu") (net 16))
 (segment (start 156.8755 101.27) (end 159.89 101.27) (width 0.25) (layer "B.Cu") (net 16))
 (segment (start 150.45 105.3) (end 150.55 105.4) (width 0.25) (layer "F.Cu") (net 17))
 (segment (start 141.25 100.875) (end 141.25 103.2995) (width 0.25) (layer "F.Cu") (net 17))
 (segment (start 141.25 103.2995) (end 143.2005 105.25) (width 0.25) (layer "F.Cu") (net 17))
 (segment (start 145.85 105.3) (end 150.45 105.3) (width 0.25) (layer "F.Cu") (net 17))
 (via (at 150.55 105.4) (size 0.8) (drill 0.4) (layers "F.Cu" "B.Cu") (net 17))
 (via (at 143.2005 105.25) (size 0.8) (drill 0.4) (layers "F.Cu" "B.Cu") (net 17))
 (via (at 145.85 105.3) (size 0.8) (drill 0.4) (layers "F.Cu" "B.Cu") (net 17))
 (segment (start 143.2005 105.25) (end 145.8 105.25) (width 0.25) (layer "B.Cu") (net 17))
 (segment (start 150.55 105.4) (end 158.3 105.4) (width 0.25) (layer "B.Cu") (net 17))
 (segment (start 158.3 105.4) (end 159.89 103.81) (width 0.25) (layer "B.Cu") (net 17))
 (segment (start 145.8 105.25) (end 145.85 105.3) (width 0.25) (layer "B.Cu") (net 17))
 (segment (start 163.25 76.97132) (end 163.25 102.95) (width 0.25) (layer "F.Cu") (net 18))
 (segment (start 163.25 102.95) (end 163.55 103.25) (width 0.25) (layer "F.Cu") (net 18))
 (segment (start 163.55 103.25) (end 163.55 106.3245) (width 0.25) (layer "F.Cu") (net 18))
 (segment (start 158.62868 72.35) (end 163.25 76.97132) (width 0.25) (layer "F.Cu") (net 18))
 (segment (start 132.473952 72.35) (end 158.62868 72.35) (width 0.25) (layer "F.Cu") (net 18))
 (segment (start 131.273952 71.15) (end 132.473952 72.35) (width 0.25) (layer "F.Cu") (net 18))
 (segment (start 91.25 99.125) (end 91.25 81.32316) (width 0.25) (layer "F.Cu") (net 18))
 (segment (start 91.25 81.32316) (end 101.42316 71.15) (width 0.25) (layer "F.Cu") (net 18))
 (segment (start 101.42316 71.15) (end 131.273952 71.15) (width 0.25) (layer "F.Cu") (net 18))
 (segment (start 163.55 106.3245) (end 163.5245 106.35) (width 0.25) (layer "F.Cu") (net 18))
 (via (at 163.5245 106.35) (size 0.8) (drill 0.4) (layers "F.Cu" "B.Cu") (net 18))
 (segment (start 159.89 106.35) (end 163.5245 106.35) (width 0.25) (layer "B.Cu") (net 18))
 (segment (start 130.963292 71.9) (end 132.163292 73.1) (width 0.25) (layer "F.Cu") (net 9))
 (segment (start 132.163292 73.1) (end 158.31802 73.1) (width 0.25) (layer "F.Cu") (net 9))
 (segment (start 162.5 108.82) (end 159.89 111.43) (width 0.25) (layer "F.Cu") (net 9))
 (segment (start 158.31802 73.1) (end 162.5 77.28198) (width 0.25) (layer "F.Cu") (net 9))
 (segment (start 110.170272 71.9) (end 130.963292 71.9) (width 0.25) (layer "F.Cu") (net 9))
 (segment (start 103.507772 78.5625) (end 110.170272 71.9) (width 0.25) (layer "F.Cu") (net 9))
 (segment (start 162.5 77.28198) (end 162.5 108.82) (width 0.25) (layer "F.Cu") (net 9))
 (segment (start 129.454728 122.9) (end 128.492228 121.9375) (width 0.25) (layer "F.Cu") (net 8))
 (segment (start 154.77868 122.9) (end 129.454728 122.9) (width 0.25) (layer "F.Cu") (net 8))
 (segment (start 156.8755 114.1245) (end 156.8755 120.80318) (width 0.25) (layer "F.Cu") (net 8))
 (segment (start 156.8755 120.80318) (end 154.77868 122.9) (width 0.25) (layer "F.Cu") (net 8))
 (via (at 156.8755 114) (size 0.8) (drill 0.4) (layers "F.Cu" "B.Cu") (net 8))
 (segment (start 156.9055 113.97) (end 156.8755 114) (width 0.25) (layer "B.Cu") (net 8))
 (segment (start 159.89 113.97) (end 156.9055 113.97) (width 0.25) (layer "B.Cu") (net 8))
 (segment (start 161.75 77.59264) (end 161.75 107.03) (width 0.25) (layer "F.Cu") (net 7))
 (segment (start 161.75 107.03) (end 159.89 108.89) (width 0.25) (layer "F.Cu") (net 7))
 (segment (start 158.00736 73.85) (end 161.75 77.59264) (width 0.25) (layer "F.Cu") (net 7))
 (segment (start 131.8 73.85) (end 158.00736 73.85) (width 0.25) (layer "F.Cu") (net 7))
 (segment (start 130.507772 79.4375) (end 130.507772 75.142228) (width 0.25) (layer "F.Cu") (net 7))
 (segment (start 130.507772 75.142228) (end 131.8 73.85) (width 0.25) (layer "F.Cu") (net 7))
 (segment (start 159.89 119.91) (end 159.89 116.51) (width 0.25) (layer "F.Cu") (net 4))
 (segment (start 140.56066 124.4) (end 155.4 124.4) (width 0.25) (layer "F.Cu") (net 4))
 (segment (start 102.492228 121.0625) (end 102.492228 134.850811) (width 0.25) (layer "F.Cu") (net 4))
 (segment (start 127.41066 137.55) (end 140.56066 124.4) (width 0.25) (layer "F.Cu") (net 4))
 (segment (start 105.191417 137.55) (end 127.41066 137.55) (width 0.25) (layer "F.Cu") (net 4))
 (segment (start 102.492228 134.850811) (end 105.191417 137.55) (width 0.25) (layer "F.Cu") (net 4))
 (segment (start 155.4 124.4) (end 159.89 119.91) (width 0.25) (layer "F.Cu") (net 4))
 (segment (start 173.395884 108.89) (end 175.13 108.89) (width 0.25) (layer "F.Cu") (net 12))
 (segment (start 165.818192 116.467692) (end 173.395884 108.89) (width 0.25) (layer "F.Cu") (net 12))
 (via (at 165.818192 116.467692) (size 0.8) (drill 0.4) (layers "F.Cu" "B.Cu") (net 12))
 (segment (start 153.7 118.3) (end 163.985884 118.3) (width 0.25) (layer "B.Cu") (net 12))
 (segment (start 151.05 117.5) (end 152.9 117.5) (width 0.25) (layer "B.Cu") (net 12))
 (segment (start 163.985884 118.3) (end 165.818192 116.467692) (width 0.25) (layer "B.Cu") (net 12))
 (segment (start 149.5 119.05) (end 151.05 117.5) (width 0.25) (layer "B.Cu") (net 12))
 (segment (start 152.9 117.5) (end 153.7 118.3) (width 0.25) (layer "B.Cu") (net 12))
 (segment (start 103.8 100) (end 103.8 96.75) (width 0.7) (layer "B.Cu") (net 2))
 (segment (start 116.35 68.75) (end 116.35 74.2) (width 0.7) (layer "B.Cu") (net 2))
 (segment (start 113.05 130.9) (end 119.55 130.9) (width 0.7) (layer "B.Cu") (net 2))
 (segment (start 168.3 117.45) (end 168.3 88.57) (width 0.7) (layer "B.Cu") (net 2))
 (segment (start 168.3 86.06) (end 168.3 88.57) (width 0.7) (layer "B.Cu") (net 2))
 (segment (start 147.25 96.8) (end 147.25 103.3) (width 0.7) (layer "B.Cu") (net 2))
 (segment (start 119.55 130.9) (end 147 130.9) (width 0.7) (layer "B.Cu") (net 2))
 (segment (start 168.3 88.57) (end 175.13 88.57) (width 0.7) (layer "B.Cu") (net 2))
 (segment (start 156.44 74.2) (end 168.3 86.06) (width 0.7) (layer "B.Cu") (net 2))
 (segment (start 147.25 103.3) (end 147.25 118.8) (width 0.7) (layer "B.Cu") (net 2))
 (segment (start 86 96.75) (end 103.8 96.75) (width 0.7) (layer "B.Cu") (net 2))
 (segment (start 154.85 130.9) (end 168.3 117.45) (width 0.7) (layer "B.Cu") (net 2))
 (segment (start 113 68.75) (end 116.35 68.75) (width 0.7) (layer "B.Cu") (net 2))
 (segment (start 103.8 83.4) (end 113 74.2) (width 0.7) (layer "B.Cu") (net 2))
 (segment (start 113 74.2) (end 116.35 74.2) (width 0.7) (layer "B.Cu") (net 2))
 (segment (start 116.35 74.2) (end 156.44 74.2) (width 0.7) (layer "B.Cu") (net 2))
 (segment (start 86 103.25) (end 86 96.75) (width 0.7) (layer "B.Cu") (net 2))
 (segment (start 147 119.05) (end 147 130.9) (width 0.7) (layer "B.Cu") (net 2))
 (segment (start 147.25 118.8) (end 147 119.05) (width 0.7) (layer "B.Cu") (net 2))
 (segment (start 147 130.9) (end 154.85 130.9) (width 0.7) (layer "B.Cu") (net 2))
 (segment (start 116.35 68.75) (end 119.5 68.75) (width 0.7) (layer "B.Cu") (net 2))
 (segment (start 103.8 96.75) (end 103.8 83.4) (width 0.7) (layer "B.Cu") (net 2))
 (segment (start 140.385 88.815) (end 129.2 100) (width 0.5) (layer "F.Cu") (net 10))
 (segment (start 140.385 87.599853) (end 140.385 88.815) (width 0.5) (layer "F.Cu") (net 10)))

